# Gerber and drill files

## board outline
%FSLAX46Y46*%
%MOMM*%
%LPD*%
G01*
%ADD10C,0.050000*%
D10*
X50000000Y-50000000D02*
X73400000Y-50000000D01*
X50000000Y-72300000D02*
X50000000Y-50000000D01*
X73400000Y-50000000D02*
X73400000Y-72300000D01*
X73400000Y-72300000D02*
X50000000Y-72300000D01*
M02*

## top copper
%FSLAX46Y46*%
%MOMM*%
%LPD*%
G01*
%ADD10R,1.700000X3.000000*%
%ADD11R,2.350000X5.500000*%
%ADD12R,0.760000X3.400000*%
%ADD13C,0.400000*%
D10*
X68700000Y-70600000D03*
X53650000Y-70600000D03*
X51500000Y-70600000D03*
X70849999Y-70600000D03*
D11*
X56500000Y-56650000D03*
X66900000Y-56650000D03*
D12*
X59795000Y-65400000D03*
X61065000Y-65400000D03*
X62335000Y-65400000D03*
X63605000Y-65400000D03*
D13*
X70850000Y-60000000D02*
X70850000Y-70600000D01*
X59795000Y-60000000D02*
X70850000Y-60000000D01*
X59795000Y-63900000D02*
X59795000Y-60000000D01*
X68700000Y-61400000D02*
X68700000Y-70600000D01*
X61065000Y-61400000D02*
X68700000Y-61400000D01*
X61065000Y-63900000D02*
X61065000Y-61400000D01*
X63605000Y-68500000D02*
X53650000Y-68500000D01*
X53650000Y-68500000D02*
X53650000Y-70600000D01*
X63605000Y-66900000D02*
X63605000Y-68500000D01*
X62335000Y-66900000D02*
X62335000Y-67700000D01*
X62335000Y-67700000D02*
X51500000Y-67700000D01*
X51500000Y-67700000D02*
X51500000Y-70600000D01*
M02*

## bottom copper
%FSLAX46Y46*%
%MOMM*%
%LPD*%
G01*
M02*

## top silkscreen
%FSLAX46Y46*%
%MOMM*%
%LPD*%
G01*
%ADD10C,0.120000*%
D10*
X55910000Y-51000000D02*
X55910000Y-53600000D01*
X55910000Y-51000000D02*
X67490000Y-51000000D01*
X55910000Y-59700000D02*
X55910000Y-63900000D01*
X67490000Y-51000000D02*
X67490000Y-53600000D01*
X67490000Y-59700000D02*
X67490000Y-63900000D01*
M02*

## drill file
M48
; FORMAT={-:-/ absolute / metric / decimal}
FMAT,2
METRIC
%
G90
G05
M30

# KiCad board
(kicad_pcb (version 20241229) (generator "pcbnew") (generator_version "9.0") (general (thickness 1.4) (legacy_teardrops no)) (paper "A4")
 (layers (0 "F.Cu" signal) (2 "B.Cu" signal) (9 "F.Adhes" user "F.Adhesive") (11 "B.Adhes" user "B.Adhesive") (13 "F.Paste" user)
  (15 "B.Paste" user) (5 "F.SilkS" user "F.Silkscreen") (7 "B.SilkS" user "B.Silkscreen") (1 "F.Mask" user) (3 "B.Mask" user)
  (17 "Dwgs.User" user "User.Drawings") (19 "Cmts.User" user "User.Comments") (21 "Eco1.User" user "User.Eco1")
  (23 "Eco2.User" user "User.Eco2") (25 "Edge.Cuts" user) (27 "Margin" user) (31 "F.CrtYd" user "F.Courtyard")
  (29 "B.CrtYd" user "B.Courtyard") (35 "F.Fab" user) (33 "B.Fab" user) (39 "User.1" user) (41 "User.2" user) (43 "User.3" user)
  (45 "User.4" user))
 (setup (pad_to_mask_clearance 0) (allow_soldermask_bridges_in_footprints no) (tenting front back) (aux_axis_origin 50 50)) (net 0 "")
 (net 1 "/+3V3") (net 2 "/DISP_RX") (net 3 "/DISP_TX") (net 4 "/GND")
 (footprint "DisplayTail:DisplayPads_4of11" (layer "F.Cu") (at 51.5 70.6)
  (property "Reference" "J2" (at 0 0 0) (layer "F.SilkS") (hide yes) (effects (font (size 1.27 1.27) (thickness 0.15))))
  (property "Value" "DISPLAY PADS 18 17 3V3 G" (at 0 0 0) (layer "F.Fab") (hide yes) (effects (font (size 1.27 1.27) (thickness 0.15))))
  (pad "3V3" smd rect (at 17.2 0) (size 1.7 3) (layers "F.Cu" "F.Mask") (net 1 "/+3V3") (thermal_bridge_angle 45))
  (pad "17" smd rect (at 2.15 0) (size 1.7 3) (layers "F.Cu" "F.Mask") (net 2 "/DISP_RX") (thermal_bridge_angle 45))
  (pad "18" smd rect (at 0 0) (size 1.7 3) (layers "F.Cu" "F.Mask") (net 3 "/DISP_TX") (thermal_bridge_angle 45))
  (pad "G" smd rect (at 19.349999 0) (size 1.7 3) (layers "F.Cu" "F.Mask") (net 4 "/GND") (thermal_bridge_angle 45)))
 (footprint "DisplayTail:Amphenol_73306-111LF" (layer "F.Cu") (at 61.7 51)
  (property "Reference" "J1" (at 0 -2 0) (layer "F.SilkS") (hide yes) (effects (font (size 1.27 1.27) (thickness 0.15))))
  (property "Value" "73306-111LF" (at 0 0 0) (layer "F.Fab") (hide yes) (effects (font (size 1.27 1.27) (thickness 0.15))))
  (fp_line (start -5.79 0) (end -5.79 2.6) (stroke (width 0.12) (type default)) (layer "F.SilkS"))
  (fp_line (start -5.79 0) (end 5.79 0) (stroke (width 0.12) (type default)) (layer "F.SilkS"))
  (fp_line (start -5.79 8.7) (end -5.79 12.9) (stroke (width 0.12) (type default)) (layer "F.SilkS"))
  (fp_line (start 5.79 0) (end 5.79 2.6) (stroke (width 0.12) (type default)) (layer "F.SilkS"))
  (fp_line (start 5.79 8.7) (end 5.79 12.9) (stroke (width 0.12) (type default)) (layer "F.SilkS"))
  (pad "" smd rect (at -5.2 5.65) (size 2.35 5.5) (layers "F.Cu" "F.Mask" "F.Paste") (thermal_bridge_angle 45))
  (pad "" smd rect (at 5.2 5.65) (size 2.35 5.5) (layers "F.Cu" "F.Mask" "F.Paste") (thermal_bridge_angle 45))
  (pad "1" smd rect (at -1.905 14.4) (size 0.76 3.4) (layers "F.Cu" "F.Mask" "F.Paste") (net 4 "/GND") (thermal_bridge_angle 45))
  (pad "2" smd rect (at -0.635 14.4) (size 0.76 3.4) (layers "F.Cu" "F.Mask" "F.Paste") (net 1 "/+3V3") (thermal_bridge_angle 45))
  (pad "3" smd rect (at 0.635 14.4) (size 0.76 3.4) (layers "F.Cu" "F.Mask" "F.Paste") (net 3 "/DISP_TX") (thermal_bridge_angle 45))
  (pad "4" smd rect (at 1.905 14.4) (size 0.76 3.4) (layers "F.Cu" "F.Mask" "F.Paste") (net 2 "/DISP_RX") (thermal_bridge_angle 45)))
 (gr_line (start 50 50) (end 73.4 50) (stroke (width 0.05) (type default)) (layer "Edge.Cuts"))
 (gr_line (start 50 72.3) (end 50 50) (stroke (width 0.05) (type default)) (layer "Edge.Cuts"))
 (gr_line (start 73.4 50) (end 73.4 72.3) (stroke (width 0.05) (type default)) (layer "Edge.Cuts"))
 (gr_line (start 73.4 72.3) (end 50 72.3) (stroke (width 0.05) (type default)) (layer "Edge.Cuts"))
 (segment (start 70.85 60) (end 70.85 70.6) (width 0.4) (layer "F.Cu") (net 4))
 (segment (start 59.795 60) (end 70.85 60) (width 0.4) (layer "F.Cu") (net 4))
 (segment (start 59.795 63.9) (end 59.795 60) (width 0.4) (layer "F.Cu") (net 4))
 (segment (start 68.7 61.4) (end 68.7 70.6) (width 0.4) (layer "F.Cu") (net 1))
 (segment (start 61.065 61.4) (end 68.7 61.4) (width 0.4) (layer "F.Cu") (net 1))
 (segment (start 61.065 63.9) (end 61.065 61.4) (width 0.4) (layer "F.Cu") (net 1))
 (segment (start 63.605 68.5) (end 53.65 68.5) (width 0.4) (layer "F.Cu") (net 2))
 (segment (start 53.65 68.5) (end 53.65 70.6) (width 0.4) (layer "F.Cu") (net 2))
 (segment (start 63.605 66.9) (end 63.605 68.5) (width 0.4) (layer "F.Cu") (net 2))
 (segment (start 62.335 66.9) (end 62.335 67.7) (width 0.4) (layer "F.Cu") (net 3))
 (segment (start 62.335 67.7) (end 51.5 67.7) (width 0.4) (layer "F.Cu") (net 3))
 (segment (start 51.5 67.7) (end 51.5 70.6) (width 0.4) (layer "F.Cu") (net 3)))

